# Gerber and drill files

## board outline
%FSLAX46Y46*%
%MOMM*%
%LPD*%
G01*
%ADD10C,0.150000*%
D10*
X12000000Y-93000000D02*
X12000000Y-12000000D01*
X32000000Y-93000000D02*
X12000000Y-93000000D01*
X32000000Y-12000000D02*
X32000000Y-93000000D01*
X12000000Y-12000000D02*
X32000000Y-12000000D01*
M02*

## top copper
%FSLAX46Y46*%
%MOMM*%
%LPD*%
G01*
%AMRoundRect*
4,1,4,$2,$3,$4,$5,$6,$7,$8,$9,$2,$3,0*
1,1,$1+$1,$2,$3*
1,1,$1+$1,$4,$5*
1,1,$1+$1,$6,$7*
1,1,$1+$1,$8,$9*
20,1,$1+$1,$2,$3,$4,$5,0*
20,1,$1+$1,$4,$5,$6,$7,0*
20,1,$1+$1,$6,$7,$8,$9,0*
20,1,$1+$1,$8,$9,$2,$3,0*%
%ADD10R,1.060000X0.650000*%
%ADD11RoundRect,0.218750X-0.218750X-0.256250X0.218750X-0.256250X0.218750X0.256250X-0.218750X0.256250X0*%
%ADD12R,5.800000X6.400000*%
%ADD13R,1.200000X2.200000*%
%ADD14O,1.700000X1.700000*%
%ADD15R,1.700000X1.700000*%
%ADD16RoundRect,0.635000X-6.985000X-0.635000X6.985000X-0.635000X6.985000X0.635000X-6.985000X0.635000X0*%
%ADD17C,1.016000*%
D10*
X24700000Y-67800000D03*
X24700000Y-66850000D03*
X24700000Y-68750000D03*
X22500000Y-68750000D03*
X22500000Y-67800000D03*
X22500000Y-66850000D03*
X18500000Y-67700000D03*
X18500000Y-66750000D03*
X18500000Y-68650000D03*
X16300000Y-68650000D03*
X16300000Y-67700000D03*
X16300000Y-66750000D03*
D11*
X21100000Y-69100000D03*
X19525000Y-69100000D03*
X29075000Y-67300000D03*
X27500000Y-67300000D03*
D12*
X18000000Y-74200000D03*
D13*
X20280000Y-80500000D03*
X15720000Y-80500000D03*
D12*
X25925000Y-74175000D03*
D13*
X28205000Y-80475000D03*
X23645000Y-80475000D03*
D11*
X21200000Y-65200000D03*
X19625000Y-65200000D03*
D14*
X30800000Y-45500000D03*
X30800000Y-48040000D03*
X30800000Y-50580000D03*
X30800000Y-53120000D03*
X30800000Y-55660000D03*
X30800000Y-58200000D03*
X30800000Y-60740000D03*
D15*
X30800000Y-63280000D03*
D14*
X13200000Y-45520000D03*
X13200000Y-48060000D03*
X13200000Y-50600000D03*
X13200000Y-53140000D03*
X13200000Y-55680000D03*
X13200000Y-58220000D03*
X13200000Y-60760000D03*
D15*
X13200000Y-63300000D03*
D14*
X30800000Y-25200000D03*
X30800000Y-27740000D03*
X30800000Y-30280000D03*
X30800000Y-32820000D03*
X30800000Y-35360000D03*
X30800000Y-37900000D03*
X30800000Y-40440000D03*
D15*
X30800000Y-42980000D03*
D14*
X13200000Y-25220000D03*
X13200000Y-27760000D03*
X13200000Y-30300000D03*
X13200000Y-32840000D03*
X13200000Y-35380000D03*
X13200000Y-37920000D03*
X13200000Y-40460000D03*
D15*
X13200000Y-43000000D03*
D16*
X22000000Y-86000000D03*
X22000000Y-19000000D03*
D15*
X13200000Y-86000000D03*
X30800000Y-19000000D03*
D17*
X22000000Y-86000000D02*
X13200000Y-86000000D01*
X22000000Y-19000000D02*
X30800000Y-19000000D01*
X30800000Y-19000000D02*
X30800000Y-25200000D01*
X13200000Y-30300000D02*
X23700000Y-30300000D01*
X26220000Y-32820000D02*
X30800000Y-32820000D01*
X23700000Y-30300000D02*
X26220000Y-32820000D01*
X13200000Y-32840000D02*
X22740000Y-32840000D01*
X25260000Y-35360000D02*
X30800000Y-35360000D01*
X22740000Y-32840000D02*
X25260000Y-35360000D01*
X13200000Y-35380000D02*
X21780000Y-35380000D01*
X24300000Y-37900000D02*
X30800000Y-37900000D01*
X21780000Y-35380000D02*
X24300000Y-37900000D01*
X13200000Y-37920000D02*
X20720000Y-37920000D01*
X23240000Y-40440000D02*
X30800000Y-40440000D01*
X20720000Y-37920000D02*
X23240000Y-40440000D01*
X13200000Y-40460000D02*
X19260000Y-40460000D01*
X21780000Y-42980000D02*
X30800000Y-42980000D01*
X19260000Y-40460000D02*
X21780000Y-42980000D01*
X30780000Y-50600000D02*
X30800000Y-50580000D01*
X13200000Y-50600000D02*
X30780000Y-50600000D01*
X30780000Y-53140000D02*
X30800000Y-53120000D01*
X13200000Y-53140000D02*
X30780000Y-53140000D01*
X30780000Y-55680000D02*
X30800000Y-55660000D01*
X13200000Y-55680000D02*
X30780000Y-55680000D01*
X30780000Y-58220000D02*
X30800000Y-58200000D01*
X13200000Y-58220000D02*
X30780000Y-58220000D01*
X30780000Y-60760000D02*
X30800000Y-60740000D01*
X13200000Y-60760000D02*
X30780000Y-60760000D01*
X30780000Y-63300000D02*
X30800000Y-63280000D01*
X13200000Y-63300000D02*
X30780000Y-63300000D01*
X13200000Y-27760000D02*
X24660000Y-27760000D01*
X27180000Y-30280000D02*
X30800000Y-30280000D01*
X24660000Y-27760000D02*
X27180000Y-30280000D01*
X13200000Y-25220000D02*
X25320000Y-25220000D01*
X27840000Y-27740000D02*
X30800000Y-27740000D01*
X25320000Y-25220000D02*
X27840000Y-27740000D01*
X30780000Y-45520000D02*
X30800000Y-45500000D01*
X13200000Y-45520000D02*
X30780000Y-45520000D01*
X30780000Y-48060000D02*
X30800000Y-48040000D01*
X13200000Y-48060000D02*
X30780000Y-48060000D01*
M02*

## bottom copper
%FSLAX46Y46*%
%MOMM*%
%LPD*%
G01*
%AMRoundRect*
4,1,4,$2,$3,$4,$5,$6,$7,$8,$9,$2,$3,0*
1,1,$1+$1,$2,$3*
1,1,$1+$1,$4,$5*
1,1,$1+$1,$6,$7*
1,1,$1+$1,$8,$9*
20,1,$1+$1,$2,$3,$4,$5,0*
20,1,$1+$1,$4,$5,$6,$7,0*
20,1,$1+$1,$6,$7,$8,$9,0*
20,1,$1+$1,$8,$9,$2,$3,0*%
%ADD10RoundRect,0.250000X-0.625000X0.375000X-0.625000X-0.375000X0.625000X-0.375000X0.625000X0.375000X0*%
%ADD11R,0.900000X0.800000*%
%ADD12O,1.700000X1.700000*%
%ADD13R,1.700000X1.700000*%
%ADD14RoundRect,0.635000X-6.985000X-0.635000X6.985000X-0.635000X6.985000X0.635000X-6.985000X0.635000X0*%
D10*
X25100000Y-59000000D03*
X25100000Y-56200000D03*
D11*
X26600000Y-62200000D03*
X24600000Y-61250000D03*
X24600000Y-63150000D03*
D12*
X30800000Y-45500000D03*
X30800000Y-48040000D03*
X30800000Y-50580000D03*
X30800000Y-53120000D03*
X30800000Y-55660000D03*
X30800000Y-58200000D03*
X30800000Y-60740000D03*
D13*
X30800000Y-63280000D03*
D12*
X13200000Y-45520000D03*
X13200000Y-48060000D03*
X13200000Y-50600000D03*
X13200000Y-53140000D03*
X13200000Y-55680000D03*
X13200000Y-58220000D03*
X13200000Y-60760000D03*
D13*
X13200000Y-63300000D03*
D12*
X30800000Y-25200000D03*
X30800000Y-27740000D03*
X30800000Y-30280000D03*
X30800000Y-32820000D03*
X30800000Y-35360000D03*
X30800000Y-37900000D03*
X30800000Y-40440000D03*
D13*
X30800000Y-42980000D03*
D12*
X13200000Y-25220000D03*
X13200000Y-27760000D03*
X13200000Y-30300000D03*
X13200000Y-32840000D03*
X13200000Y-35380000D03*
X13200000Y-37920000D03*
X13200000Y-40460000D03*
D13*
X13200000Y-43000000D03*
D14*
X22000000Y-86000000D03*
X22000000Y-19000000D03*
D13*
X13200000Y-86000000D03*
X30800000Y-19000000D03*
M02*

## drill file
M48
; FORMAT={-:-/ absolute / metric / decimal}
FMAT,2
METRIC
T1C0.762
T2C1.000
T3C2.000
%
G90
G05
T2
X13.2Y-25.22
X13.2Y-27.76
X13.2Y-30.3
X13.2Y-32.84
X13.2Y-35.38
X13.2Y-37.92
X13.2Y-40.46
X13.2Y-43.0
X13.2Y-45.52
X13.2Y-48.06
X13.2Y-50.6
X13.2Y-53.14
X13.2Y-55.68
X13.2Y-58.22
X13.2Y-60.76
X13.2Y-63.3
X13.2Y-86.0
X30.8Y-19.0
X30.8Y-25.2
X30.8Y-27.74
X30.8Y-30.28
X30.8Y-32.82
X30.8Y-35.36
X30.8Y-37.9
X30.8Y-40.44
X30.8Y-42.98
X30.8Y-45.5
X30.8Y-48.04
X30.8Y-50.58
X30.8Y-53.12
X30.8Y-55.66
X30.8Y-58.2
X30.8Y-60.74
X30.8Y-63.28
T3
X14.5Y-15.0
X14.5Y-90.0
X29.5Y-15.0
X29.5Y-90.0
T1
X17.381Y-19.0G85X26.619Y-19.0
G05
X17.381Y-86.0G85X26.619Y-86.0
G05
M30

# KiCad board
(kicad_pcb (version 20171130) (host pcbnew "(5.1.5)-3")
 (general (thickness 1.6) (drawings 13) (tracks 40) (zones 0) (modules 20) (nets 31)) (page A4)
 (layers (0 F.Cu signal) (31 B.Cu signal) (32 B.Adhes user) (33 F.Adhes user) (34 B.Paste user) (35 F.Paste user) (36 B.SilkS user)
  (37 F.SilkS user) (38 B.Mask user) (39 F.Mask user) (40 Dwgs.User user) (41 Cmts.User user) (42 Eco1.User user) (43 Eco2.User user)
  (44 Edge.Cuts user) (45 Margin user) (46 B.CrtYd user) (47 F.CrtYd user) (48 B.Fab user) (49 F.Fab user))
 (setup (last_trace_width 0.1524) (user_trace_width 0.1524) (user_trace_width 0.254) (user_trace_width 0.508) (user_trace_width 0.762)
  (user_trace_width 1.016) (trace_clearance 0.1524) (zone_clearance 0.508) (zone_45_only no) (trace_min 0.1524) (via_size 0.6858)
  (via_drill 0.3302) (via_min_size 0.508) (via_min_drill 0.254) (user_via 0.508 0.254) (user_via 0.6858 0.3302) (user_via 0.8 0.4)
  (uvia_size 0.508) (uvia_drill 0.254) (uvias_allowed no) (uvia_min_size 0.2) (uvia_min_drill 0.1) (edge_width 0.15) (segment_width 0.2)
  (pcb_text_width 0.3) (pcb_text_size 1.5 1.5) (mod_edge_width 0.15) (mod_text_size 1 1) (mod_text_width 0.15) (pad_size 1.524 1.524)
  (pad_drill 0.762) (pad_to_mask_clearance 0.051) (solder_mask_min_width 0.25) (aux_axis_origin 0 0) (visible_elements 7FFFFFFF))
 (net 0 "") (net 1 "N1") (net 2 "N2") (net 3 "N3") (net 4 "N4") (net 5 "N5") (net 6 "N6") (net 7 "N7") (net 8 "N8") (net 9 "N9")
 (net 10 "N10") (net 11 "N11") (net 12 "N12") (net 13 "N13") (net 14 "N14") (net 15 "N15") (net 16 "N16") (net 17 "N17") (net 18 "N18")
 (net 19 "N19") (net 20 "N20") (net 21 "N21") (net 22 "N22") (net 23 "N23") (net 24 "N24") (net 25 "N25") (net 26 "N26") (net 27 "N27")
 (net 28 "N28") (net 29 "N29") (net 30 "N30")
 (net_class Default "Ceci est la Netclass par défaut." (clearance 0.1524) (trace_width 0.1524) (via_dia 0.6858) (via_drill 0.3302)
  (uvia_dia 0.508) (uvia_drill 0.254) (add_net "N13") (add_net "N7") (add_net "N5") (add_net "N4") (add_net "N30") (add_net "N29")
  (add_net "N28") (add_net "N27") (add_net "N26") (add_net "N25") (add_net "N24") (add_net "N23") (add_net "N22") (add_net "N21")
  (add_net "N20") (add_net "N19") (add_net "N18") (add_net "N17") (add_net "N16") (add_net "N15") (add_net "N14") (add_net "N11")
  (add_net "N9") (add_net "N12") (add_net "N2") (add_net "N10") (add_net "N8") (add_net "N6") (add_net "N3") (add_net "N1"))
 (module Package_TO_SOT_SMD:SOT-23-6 (layer F.Cu) (at 23.6 67.8)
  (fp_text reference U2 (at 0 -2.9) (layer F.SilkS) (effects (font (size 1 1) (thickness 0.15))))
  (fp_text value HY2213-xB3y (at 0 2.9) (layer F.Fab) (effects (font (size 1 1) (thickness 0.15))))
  (pad 5 smd rect (at 1.1 0) (size 1.06 0.65) (layers F.Cu F.Paste F.Mask) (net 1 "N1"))
  (pad 6 smd rect (at 1.1 -0.95) (size 1.06 0.65) (layers F.Cu F.Paste F.Mask) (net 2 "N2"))
  (pad 4 smd rect (at 1.1 0.95) (size 1.06 0.65) (layers F.Cu F.Paste F.Mask) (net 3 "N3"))
  (pad 3 smd rect (at -1.1 0.95) (size 1.06 0.65) (layers F.Cu F.Paste F.Mask) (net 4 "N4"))
  (pad 2 smd rect (at -1.1 0) (size 1.06 0.65) (layers F.Cu F.Paste F.Mask) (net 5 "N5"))
  (pad 1 smd rect (at -1.1 -0.95) (size 1.06 0.65) (layers F.Cu F.Paste F.Mask) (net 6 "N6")))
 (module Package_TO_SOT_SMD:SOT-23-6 (layer F.Cu) (at 17.4 67.7)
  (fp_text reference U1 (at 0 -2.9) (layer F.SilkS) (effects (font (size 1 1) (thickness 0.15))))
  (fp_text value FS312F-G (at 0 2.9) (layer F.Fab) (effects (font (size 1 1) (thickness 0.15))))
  (pad 5 smd rect (at 1.1 0) (size 1.06 0.65) (layers F.Cu F.Paste F.Mask) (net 5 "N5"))
  (pad 6 smd rect (at 1.1 -0.95) (size 1.06 0.65) (layers F.Cu F.Paste F.Mask) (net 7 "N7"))
  (pad 4 smd rect (at 1.1 0.95) (size 1.06 0.65) (layers F.Cu F.Paste F.Mask) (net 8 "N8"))
  (pad 3 smd rect (at -1.1 0.95) (size 1.06 0.65) (layers F.Cu F.Paste F.Mask) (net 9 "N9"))
  (pad 2 smd rect (at -1.1 0) (size 1.06 0.65) (layers F.Cu F.Paste F.Mask) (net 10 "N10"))
  (pad 1 smd rect (at -1.1 -0.95) (size 1.06 0.65) (layers F.Cu F.Paste F.Mask) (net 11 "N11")))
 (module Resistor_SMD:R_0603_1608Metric (layer F.Cu) (at 20.3125 69.1)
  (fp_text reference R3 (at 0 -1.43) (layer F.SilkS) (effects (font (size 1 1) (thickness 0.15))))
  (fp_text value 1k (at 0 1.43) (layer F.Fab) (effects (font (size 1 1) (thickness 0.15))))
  (pad 2 smd roundrect (at 0.7875 0) (size 0.875 0.95) (layers F.Cu F.Paste F.Mask) (roundrect_rratio 0.25) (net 10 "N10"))
  (pad 1 smd roundrect (at -0.7875 0) (size 0.875 0.95) (layers F.Cu F.Paste F.Mask) (roundrect_rratio 0.25) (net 4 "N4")))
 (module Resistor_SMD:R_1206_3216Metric (layer B.Cu) (at 25.1 57.6 270)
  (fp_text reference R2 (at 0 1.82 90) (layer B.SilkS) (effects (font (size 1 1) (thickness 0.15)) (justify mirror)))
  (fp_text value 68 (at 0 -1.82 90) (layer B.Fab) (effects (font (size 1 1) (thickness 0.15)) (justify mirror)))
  (pad 2 smd roundrect (at 1.4 0 270) (size 1.25 1.75) (layers B.Cu B.Paste B.Mask) (roundrect_rratio 0.2) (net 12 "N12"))
  (pad 1 smd roundrect (at -1.4 0 270) (size 1.25 1.75) (layers B.Cu B.Paste B.Mask) (roundrect_rratio 0.2) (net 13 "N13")))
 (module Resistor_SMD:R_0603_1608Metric (layer F.Cu) (at 28.2875 67.3)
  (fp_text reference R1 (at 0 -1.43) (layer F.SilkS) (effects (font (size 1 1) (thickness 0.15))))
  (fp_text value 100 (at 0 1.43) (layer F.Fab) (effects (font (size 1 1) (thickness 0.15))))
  (pad 2 smd roundrect (at 0.7875 0) (size 0.875 0.95) (layers F.Cu F.Paste F.Mask) (roundrect_rratio 0.25) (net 13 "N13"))
  (pad 1 smd roundrect (at -0.7875 0) (size 0.875 0.95) (layers F.Cu F.Paste F.Mask) (roundrect_rratio 0.25) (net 5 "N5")))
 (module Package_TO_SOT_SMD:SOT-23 (layer B.Cu) (at 25.6 62.2)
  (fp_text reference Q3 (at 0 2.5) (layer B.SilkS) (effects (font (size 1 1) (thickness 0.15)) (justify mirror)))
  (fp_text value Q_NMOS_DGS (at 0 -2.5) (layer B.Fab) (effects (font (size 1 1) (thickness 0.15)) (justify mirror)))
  (pad 3 smd rect (at 1 0) (size 0.9 0.8) (layers B.Cu B.Paste B.Mask) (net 4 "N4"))
  (pad 2 smd rect (at -1 -0.95) (size 0.9 0.8) (layers B.Cu B.Paste B.Mask) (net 2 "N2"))
  (pad 1 smd rect (at -1 0.95) (size 0.9 0.8) (layers B.Cu B.Paste B.Mask) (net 12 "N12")))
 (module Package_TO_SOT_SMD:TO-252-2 (layer F.Cu) (at 18 76.3 90)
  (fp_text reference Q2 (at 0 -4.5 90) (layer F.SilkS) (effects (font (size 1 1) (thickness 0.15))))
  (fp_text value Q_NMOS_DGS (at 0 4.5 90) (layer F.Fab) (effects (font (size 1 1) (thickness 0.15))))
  (pad "" smd rect (at 0.425 1.525 90) (size 3.05 2.75) (layers F.Paste))
  (pad "" smd rect (at 3.775 -1.525 90) (size 3.05 2.75) (layers F.Paste))
  (pad "" smd rect (at 0.425 -1.525 90) (size 3.05 2.75) (layers F.Paste))
  (pad "" smd rect (at 3.775 1.525 90) (size 3.05 2.75) (layers F.Paste))
  (pad 2 smd rect (at 2.1 0 90) (size 6.4 5.8) (layers F.Cu F.Mask) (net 9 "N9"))
  (pad 3 smd rect (at -4.2 2.28 90) (size 2.2 1.2) (layers F.Cu F.Paste F.Mask) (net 4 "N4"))
  (pad 1 smd rect (at -4.2 -2.28 90) (size 2.2 1.2) (layers F.Cu F.Paste F.Mask) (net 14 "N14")))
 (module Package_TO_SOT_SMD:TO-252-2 (layer F.Cu) (at 25.925 76.275 90)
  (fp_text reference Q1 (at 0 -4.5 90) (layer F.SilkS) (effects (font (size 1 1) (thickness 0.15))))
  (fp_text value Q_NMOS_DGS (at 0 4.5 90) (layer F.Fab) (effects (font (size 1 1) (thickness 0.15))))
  (pad "" smd rect (at 0.425 1.525 90) (size 3.05 2.75) (layers F.Paste))
  (pad "" smd rect (at 3.775 -1.525 90) (size 3.05 2.75) (layers F.Paste))
  (pad "" smd rect (at 0.425 -1.525 90) (size 3.05 2.75) (layers F.Paste))
  (pad "" smd rect (at 3.775 1.525 90) (size 3.05 2.75) (layers F.Paste))
  (pad 2 smd rect (at 2.1 0 90) (size 6.4 5.8) (layers F.Cu F.Mask) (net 11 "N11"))
  (pad 3 smd rect (at -4.2 2.28 90) (size 2.2 1.2) (layers F.Cu F.Paste F.Mask) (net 7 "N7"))
  (pad 1 smd rect (at -4.2 -2.28 90) (size 2.2 1.2) (layers F.Cu F.Paste F.Mask) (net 14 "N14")))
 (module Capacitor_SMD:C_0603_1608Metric (layer F.Cu) (at 20.4125 65.2)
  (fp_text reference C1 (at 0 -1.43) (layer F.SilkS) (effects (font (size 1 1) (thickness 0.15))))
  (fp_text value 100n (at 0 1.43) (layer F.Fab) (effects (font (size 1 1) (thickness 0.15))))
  (pad 2 smd roundrect (at 0.7875 0) (size 0.875 0.95) (layers F.Cu F.Paste F.Mask) (roundrect_rratio 0.25) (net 7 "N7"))
  (pad 1 smd roundrect (at -0.7875 0) (size 0.875 0.95) (layers F.Cu F.Paste F.Mask) (roundrect_rratio 0.25) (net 5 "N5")))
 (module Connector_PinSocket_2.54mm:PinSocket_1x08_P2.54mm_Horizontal (layer F.Cu) (at 30.8 63.28 180)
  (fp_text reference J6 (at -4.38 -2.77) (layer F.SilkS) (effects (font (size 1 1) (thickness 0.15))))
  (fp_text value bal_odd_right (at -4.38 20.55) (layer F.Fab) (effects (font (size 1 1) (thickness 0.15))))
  (pad 8 thru_hole oval (at 0 17.78 180) (size 1.7 1.7) (drill 1) (layers *.Cu *.Mask) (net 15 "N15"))
  (pad 7 thru_hole oval (at 0 15.24 180) (size 1.7 1.7) (drill 1) (layers *.Cu *.Mask) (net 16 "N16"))
  (pad 6 thru_hole oval (at 0 12.7 180) (size 1.7 1.7) (drill 1) (layers *.Cu *.Mask) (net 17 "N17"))
  (pad 5 thru_hole oval (at 0 10.16 180) (size 1.7 1.7) (drill 1) (layers *.Cu *.Mask) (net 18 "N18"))
  (pad 4 thru_hole oval (at 0 7.62 180) (size 1.7 1.7) (drill 1) (layers *.Cu *.Mask) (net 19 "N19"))
  (pad 3 thru_hole oval (at 0 5.08 180) (size 1.7 1.7) (drill 1) (layers *.Cu *.Mask) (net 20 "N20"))
  (pad 2 thru_hole oval (at 0 2.54 180) (size 1.7 1.7) (drill 1) (layers *.Cu *.Mask) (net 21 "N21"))
  (pad 1 thru_hole rect (at 0 0 180) (size 1.7 1.7) (drill 1) (layers *.Cu *.Mask) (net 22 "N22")))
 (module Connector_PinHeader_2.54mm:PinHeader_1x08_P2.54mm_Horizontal (layer F.Cu) (at 13.2 63.3 180)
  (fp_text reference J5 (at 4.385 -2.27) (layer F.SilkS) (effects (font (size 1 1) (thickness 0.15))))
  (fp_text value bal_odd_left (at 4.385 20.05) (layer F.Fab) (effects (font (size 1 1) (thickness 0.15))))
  (pad 8 thru_hole oval (at 0 17.78 180) (size 1.7 1.7) (drill 1) (layers *.Cu *.Mask) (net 15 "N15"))
  (pad 7 thru_hole oval (at 0 15.24 180) (size 1.7 1.7) (drill 1) (layers *.Cu *.Mask) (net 16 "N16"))
  (pad 6 thru_hole oval (at 0 12.7 180) (size 1.7 1.7) (drill 1) (layers *.Cu *.Mask) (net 17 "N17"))
  (pad 5 thru_hole oval (at 0 10.16 180) (size 1.7 1.7) (drill 1) (layers *.Cu *.Mask) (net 18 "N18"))
  (pad 4 thru_hole oval (at 0 7.62 180) (size 1.7 1.7) (drill 1) (layers *.Cu *.Mask) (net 19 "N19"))
  (pad 3 thru_hole oval (at 0 5.08 180) (size 1.7 1.7) (drill 1) (layers *.Cu *.Mask) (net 20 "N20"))
  (pad 2 thru_hole oval (at 0 2.54 180) (size 1.7 1.7) (drill 1) (layers *.Cu *.Mask) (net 21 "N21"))
  (pad 1 thru_hole rect (at 0 0 180) (size 1.7 1.7) (drill 1) (layers *.Cu *.Mask) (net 22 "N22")))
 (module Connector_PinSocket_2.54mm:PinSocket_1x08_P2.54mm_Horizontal (layer F.Cu) (at 30.8 42.98 180)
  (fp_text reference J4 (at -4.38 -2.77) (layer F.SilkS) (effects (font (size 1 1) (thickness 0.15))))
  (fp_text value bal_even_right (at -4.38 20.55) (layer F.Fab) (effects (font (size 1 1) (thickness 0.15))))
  (pad 8 thru_hole oval (at 0 17.78 180) (size 1.7 1.7) (drill 1) (layers *.Cu *.Mask) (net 13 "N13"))
  (pad 7 thru_hole oval (at 0 15.24 180) (size 1.7 1.7) (drill 1) (layers *.Cu *.Mask) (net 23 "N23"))
  (pad 6 thru_hole oval (at 0 12.7 180) (size 1.7 1.7) (drill 1) (layers *.Cu *.Mask) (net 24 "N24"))
  (pad 5 thru_hole oval (at 0 10.16 180) (size 1.7 1.7) (drill 1) (layers *.Cu *.Mask) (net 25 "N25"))
  (pad 4 thru_hole oval (at 0 7.62 180) (size 1.7 1.7) (drill 1) (layers *.Cu *.Mask) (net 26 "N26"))
  (pad 3 thru_hole oval (at 0 5.08 180) (size 1.7 1.7) (drill 1) (layers *.Cu *.Mask) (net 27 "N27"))
  (pad 2 thru_hole oval (at 0 2.54 180) (size 1.7 1.7) (drill 1) (layers *.Cu *.Mask) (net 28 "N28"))
  (pad 1 thru_hole rect (at 0 0 180) (size 1.7 1.7) (drill 1) (layers *.Cu *.Mask) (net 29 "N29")))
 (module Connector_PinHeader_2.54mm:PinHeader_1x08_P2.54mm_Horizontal (layer F.Cu) (at 13.2 43 180)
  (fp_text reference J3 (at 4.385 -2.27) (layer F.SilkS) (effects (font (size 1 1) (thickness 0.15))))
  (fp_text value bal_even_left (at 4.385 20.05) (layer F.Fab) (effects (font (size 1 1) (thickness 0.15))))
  (pad 8 thru_hole oval (at 0 17.78 180) (size 1.7 1.7) (drill 1) (layers *.Cu *.Mask) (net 23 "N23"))
  (pad 7 thru_hole oval (at 0 15.24 180) (size 1.7 1.7) (drill 1) (layers *.Cu *.Mask) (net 24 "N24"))
  (pad 6 thru_hole oval (at 0 12.7 180) (size 1.7 1.7) (drill 1) (layers *.Cu *.Mask) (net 25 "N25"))
  (pad 5 thru_hole oval (at 0 10.16 180) (size 1.7 1.7) (drill 1) (layers *.Cu *.Mask) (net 26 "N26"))
  (pad 4 thru_hole oval (at 0 7.62 180) (size 1.7 1.7) (drill 1) (layers *.Cu *.Mask) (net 27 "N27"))
  (pad 3 thru_hole oval (at 0 5.08 180) (size 1.7 1.7) (drill 1) (layers *.Cu *.Mask) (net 28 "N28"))
  (pad 2 thru_hole oval (at 0 2.54 180) (size 1.7 1.7) (drill 1) (layers *.Cu *.Mask) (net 29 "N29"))
  (pad 1 thru_hole rect (at 0 0 180) (size 1.7 1.7) (drill 1) (layers *.Cu *.Mask) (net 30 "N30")))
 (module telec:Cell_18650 (layer F.Cu) (at 22 19)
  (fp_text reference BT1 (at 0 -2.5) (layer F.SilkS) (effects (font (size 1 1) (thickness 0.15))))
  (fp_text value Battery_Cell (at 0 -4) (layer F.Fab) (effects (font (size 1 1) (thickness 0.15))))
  (pad 2 thru_hole roundrect (at 0 67) (size 15.24 2.54) (drill oval 10 0.762) (layers *.Cu *.Mask) (roundrect_rratio 0.25) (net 7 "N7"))
  (pad 1 thru_hole roundrect (at 0 0) (size 15.24 2.54) (drill oval 10 0.762) (layers *.Cu *.Mask) (roundrect_rratio 0.25) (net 13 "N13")))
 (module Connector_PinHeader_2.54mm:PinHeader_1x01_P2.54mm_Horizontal (layer F.Cu) (at 13.2 86 180)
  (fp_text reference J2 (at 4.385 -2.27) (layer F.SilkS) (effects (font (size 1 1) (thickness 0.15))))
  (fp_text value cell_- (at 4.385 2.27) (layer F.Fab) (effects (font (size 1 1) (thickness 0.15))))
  (pad 1 thru_hole rect (at 0 0 180) (size 1.7 1.7) (drill 1) (layers *.Cu *.Mask) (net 4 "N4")))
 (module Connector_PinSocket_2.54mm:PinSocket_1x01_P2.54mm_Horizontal (layer F.Cu) (at 30.8 19 180)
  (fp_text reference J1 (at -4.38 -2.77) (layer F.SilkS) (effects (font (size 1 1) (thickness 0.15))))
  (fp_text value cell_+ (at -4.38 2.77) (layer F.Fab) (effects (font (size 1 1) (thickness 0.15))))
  (pad 1 thru_hole rect (at 0 0 180) (size 1.7 1.7) (drill 1) (layers *.Cu *.Mask) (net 13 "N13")))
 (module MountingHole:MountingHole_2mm (layer F.Cu) (at 14.5 90)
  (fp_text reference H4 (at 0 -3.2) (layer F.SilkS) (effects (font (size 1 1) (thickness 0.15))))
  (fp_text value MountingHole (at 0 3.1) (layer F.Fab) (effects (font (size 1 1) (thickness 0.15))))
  (pad "" np_thru_hole circle (at 0 0) (size 2 2) (drill 2) (layers *.Cu *.Mask)))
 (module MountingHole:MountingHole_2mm (layer F.Cu) (at 29.5 90)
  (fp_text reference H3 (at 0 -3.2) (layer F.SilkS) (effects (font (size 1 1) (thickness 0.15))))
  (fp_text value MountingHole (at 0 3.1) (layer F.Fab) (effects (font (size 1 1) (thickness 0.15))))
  (pad "" np_thru_hole circle (at 0 0) (size 2 2) (drill 2) (layers *.Cu *.Mask)))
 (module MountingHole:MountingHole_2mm (layer F.Cu) (at 29.5 15)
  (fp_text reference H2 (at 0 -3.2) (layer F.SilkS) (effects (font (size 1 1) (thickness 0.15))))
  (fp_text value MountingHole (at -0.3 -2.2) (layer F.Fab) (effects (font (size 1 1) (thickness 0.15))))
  (pad "" np_thru_hole circle (at 0 0) (size 2 2) (drill 2) (layers *.Cu *.Mask)))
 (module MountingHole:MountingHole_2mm (layer F.Cu) (at 14.5 15)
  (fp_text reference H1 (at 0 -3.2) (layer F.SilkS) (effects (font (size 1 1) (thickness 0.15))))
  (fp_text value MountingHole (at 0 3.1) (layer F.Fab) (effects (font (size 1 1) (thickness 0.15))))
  (pad "" np_thru_hole circle (at 0 0) (size 2 2) (drill 2) (layers *.Cu *.Mask)))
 (gr_line (start 12 93) (end 12 12) (layer Edge.Cuts) (width 0.15))
 (gr_line (start 32 93) (end 12 93) (layer Edge.Cuts) (width 0.15))
 (gr_line (start 32 12) (end 32 93) (layer Edge.Cuts) (width 0.15))
 (gr_line (start 12 12) (end 32 12) (layer Edge.Cuts) (width 0.15))
 (segment (start 22 86) (end 13.2 86) (width 1.016) (layer F.Cu) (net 7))
 (segment (start 22 19) (end 30.8 19) (width 1.016) (layer F.Cu) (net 13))
 (segment (start 30.8 19) (end 30.8 25.2) (width 1.016) (layer F.Cu) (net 13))
 (segment (start 13.2 30.3) (end 23.7 30.3) (width 1.016) (layer F.Cu) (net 25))
 (segment (start 26.22 32.82) (end 30.8 32.82) (width 1.016) (layer F.Cu) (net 25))
 (segment (start 23.7 30.3) (end 26.22 32.82) (width 1.016) (layer F.Cu) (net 25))
 (segment (start 13.2 32.84) (end 22.74 32.84) (width 1.016) (layer F.Cu) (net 26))
 (segment (start 25.26 35.36) (end 30.8 35.36) (width 1.016) (layer F.Cu) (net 26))
 (segment (start 22.74 32.84) (end 25.26 35.36) (width 1.016) (layer F.Cu) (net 26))
 (segment (start 13.2 35.38) (end 21.78 35.38) (width 1.016) (layer F.Cu) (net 27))
 (segment (start 24.3 37.9) (end 30.8 37.9) (width 1.016) (layer F.Cu) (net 27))
 (segment (start 21.78 35.38) (end 24.3 37.9) (width 1.016) (layer F.Cu) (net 27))
 (segment (start 13.2 37.92) (end 20.72 37.92) (width 1.016) (layer F.Cu) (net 28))
 (segment (start 23.24 40.44) (end 30.8 40.44) (width 1.016) (layer F.Cu) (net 28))
 (segment (start 20.72 37.92) (end 23.24 40.44) (width 1.016) (layer F.Cu) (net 28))
 (segment (start 13.2 40.46) (end 19.26 40.46) (width 1.016) (layer F.Cu) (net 29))
 (segment (start 21.78 42.98) (end 30.8 42.98) (width 1.016) (layer F.Cu) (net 29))
 (segment (start 19.26 40.46) (end 21.78 42.98) (width 1.016) (layer F.Cu) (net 29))
 (segment (start 30.78 50.6) (end 30.8 50.58) (width 1.016) (layer F.Cu) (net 17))
 (segment (start 13.2 50.6) (end 30.78 50.6) (width 1.016) (layer F.Cu) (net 17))
 (segment (start 30.78 53.14) (end 30.8 53.12) (width 1.016) (layer F.Cu) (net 18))
 (segment (start 13.2 53.14) (end 30.78 53.14) (width 1.016) (layer F.Cu) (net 18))
 (segment (start 30.78 55.68) (end 30.8 55.66) (width 1.016) (layer F.Cu) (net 19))
 (segment (start 13.2 55.68) (end 30.78 55.68) (width 1.016) (layer F.Cu) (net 19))
 (segment (start 30.78 58.22) (end 30.8 58.2) (width 1.016) (layer F.Cu) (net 20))
 (segment (start 13.2 58.22) (end 30.78 58.22) (width 1.016) (layer F.Cu) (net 20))
 (segment (start 30.78 60.76) (end 30.8 60.74) (width 1.016) (layer F.Cu) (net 21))
 (segment (start 13.2 60.76) (end 30.78 60.76) (width 1.016) (layer F.Cu) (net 21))
 (segment (start 30.78 63.3) (end 30.8 63.28) (width 1.016) (layer F.Cu) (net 22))
 (segment (start 13.2 63.3) (end 30.78 63.3) (width 1.016) (layer F.Cu) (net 22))
 (segment (start 13.2 27.76) (end 24.66 27.76) (width 1.016) (layer F.Cu) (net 24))
 (segment (start 27.18 30.28) (end 30.8 30.28) (width 1.016) (layer F.Cu) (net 24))
 (segment (start 24.66 27.76) (end 27.18 30.28) (width 1.016) (layer F.Cu) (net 24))
 (segment (start 13.2 25.22) (end 25.32 25.22) (width 1.016) (layer F.Cu) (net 23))
 (segment (start 27.84 27.74) (end 30.8 27.74) (width 1.016) (layer F.Cu) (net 23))
 (segment (start 25.32 25.22) (end 27.84 27.74) (width 1.016) (layer F.Cu) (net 23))
 (segment (start 30.78 45.52) (end 30.8 45.5) (width 1.016) (layer F.Cu) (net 15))
 (segment (start 13.2 45.52) (end 30.78 45.52) (width 1.016) (layer F.Cu) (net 15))
 (segment (start 30.78 48.06) (end 30.8 48.04) (width 1.016) (layer F.Cu) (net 16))
 (segment (start 13.2 48.06) (end 30.78 48.06) (width 1.016) (layer F.Cu) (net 16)))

